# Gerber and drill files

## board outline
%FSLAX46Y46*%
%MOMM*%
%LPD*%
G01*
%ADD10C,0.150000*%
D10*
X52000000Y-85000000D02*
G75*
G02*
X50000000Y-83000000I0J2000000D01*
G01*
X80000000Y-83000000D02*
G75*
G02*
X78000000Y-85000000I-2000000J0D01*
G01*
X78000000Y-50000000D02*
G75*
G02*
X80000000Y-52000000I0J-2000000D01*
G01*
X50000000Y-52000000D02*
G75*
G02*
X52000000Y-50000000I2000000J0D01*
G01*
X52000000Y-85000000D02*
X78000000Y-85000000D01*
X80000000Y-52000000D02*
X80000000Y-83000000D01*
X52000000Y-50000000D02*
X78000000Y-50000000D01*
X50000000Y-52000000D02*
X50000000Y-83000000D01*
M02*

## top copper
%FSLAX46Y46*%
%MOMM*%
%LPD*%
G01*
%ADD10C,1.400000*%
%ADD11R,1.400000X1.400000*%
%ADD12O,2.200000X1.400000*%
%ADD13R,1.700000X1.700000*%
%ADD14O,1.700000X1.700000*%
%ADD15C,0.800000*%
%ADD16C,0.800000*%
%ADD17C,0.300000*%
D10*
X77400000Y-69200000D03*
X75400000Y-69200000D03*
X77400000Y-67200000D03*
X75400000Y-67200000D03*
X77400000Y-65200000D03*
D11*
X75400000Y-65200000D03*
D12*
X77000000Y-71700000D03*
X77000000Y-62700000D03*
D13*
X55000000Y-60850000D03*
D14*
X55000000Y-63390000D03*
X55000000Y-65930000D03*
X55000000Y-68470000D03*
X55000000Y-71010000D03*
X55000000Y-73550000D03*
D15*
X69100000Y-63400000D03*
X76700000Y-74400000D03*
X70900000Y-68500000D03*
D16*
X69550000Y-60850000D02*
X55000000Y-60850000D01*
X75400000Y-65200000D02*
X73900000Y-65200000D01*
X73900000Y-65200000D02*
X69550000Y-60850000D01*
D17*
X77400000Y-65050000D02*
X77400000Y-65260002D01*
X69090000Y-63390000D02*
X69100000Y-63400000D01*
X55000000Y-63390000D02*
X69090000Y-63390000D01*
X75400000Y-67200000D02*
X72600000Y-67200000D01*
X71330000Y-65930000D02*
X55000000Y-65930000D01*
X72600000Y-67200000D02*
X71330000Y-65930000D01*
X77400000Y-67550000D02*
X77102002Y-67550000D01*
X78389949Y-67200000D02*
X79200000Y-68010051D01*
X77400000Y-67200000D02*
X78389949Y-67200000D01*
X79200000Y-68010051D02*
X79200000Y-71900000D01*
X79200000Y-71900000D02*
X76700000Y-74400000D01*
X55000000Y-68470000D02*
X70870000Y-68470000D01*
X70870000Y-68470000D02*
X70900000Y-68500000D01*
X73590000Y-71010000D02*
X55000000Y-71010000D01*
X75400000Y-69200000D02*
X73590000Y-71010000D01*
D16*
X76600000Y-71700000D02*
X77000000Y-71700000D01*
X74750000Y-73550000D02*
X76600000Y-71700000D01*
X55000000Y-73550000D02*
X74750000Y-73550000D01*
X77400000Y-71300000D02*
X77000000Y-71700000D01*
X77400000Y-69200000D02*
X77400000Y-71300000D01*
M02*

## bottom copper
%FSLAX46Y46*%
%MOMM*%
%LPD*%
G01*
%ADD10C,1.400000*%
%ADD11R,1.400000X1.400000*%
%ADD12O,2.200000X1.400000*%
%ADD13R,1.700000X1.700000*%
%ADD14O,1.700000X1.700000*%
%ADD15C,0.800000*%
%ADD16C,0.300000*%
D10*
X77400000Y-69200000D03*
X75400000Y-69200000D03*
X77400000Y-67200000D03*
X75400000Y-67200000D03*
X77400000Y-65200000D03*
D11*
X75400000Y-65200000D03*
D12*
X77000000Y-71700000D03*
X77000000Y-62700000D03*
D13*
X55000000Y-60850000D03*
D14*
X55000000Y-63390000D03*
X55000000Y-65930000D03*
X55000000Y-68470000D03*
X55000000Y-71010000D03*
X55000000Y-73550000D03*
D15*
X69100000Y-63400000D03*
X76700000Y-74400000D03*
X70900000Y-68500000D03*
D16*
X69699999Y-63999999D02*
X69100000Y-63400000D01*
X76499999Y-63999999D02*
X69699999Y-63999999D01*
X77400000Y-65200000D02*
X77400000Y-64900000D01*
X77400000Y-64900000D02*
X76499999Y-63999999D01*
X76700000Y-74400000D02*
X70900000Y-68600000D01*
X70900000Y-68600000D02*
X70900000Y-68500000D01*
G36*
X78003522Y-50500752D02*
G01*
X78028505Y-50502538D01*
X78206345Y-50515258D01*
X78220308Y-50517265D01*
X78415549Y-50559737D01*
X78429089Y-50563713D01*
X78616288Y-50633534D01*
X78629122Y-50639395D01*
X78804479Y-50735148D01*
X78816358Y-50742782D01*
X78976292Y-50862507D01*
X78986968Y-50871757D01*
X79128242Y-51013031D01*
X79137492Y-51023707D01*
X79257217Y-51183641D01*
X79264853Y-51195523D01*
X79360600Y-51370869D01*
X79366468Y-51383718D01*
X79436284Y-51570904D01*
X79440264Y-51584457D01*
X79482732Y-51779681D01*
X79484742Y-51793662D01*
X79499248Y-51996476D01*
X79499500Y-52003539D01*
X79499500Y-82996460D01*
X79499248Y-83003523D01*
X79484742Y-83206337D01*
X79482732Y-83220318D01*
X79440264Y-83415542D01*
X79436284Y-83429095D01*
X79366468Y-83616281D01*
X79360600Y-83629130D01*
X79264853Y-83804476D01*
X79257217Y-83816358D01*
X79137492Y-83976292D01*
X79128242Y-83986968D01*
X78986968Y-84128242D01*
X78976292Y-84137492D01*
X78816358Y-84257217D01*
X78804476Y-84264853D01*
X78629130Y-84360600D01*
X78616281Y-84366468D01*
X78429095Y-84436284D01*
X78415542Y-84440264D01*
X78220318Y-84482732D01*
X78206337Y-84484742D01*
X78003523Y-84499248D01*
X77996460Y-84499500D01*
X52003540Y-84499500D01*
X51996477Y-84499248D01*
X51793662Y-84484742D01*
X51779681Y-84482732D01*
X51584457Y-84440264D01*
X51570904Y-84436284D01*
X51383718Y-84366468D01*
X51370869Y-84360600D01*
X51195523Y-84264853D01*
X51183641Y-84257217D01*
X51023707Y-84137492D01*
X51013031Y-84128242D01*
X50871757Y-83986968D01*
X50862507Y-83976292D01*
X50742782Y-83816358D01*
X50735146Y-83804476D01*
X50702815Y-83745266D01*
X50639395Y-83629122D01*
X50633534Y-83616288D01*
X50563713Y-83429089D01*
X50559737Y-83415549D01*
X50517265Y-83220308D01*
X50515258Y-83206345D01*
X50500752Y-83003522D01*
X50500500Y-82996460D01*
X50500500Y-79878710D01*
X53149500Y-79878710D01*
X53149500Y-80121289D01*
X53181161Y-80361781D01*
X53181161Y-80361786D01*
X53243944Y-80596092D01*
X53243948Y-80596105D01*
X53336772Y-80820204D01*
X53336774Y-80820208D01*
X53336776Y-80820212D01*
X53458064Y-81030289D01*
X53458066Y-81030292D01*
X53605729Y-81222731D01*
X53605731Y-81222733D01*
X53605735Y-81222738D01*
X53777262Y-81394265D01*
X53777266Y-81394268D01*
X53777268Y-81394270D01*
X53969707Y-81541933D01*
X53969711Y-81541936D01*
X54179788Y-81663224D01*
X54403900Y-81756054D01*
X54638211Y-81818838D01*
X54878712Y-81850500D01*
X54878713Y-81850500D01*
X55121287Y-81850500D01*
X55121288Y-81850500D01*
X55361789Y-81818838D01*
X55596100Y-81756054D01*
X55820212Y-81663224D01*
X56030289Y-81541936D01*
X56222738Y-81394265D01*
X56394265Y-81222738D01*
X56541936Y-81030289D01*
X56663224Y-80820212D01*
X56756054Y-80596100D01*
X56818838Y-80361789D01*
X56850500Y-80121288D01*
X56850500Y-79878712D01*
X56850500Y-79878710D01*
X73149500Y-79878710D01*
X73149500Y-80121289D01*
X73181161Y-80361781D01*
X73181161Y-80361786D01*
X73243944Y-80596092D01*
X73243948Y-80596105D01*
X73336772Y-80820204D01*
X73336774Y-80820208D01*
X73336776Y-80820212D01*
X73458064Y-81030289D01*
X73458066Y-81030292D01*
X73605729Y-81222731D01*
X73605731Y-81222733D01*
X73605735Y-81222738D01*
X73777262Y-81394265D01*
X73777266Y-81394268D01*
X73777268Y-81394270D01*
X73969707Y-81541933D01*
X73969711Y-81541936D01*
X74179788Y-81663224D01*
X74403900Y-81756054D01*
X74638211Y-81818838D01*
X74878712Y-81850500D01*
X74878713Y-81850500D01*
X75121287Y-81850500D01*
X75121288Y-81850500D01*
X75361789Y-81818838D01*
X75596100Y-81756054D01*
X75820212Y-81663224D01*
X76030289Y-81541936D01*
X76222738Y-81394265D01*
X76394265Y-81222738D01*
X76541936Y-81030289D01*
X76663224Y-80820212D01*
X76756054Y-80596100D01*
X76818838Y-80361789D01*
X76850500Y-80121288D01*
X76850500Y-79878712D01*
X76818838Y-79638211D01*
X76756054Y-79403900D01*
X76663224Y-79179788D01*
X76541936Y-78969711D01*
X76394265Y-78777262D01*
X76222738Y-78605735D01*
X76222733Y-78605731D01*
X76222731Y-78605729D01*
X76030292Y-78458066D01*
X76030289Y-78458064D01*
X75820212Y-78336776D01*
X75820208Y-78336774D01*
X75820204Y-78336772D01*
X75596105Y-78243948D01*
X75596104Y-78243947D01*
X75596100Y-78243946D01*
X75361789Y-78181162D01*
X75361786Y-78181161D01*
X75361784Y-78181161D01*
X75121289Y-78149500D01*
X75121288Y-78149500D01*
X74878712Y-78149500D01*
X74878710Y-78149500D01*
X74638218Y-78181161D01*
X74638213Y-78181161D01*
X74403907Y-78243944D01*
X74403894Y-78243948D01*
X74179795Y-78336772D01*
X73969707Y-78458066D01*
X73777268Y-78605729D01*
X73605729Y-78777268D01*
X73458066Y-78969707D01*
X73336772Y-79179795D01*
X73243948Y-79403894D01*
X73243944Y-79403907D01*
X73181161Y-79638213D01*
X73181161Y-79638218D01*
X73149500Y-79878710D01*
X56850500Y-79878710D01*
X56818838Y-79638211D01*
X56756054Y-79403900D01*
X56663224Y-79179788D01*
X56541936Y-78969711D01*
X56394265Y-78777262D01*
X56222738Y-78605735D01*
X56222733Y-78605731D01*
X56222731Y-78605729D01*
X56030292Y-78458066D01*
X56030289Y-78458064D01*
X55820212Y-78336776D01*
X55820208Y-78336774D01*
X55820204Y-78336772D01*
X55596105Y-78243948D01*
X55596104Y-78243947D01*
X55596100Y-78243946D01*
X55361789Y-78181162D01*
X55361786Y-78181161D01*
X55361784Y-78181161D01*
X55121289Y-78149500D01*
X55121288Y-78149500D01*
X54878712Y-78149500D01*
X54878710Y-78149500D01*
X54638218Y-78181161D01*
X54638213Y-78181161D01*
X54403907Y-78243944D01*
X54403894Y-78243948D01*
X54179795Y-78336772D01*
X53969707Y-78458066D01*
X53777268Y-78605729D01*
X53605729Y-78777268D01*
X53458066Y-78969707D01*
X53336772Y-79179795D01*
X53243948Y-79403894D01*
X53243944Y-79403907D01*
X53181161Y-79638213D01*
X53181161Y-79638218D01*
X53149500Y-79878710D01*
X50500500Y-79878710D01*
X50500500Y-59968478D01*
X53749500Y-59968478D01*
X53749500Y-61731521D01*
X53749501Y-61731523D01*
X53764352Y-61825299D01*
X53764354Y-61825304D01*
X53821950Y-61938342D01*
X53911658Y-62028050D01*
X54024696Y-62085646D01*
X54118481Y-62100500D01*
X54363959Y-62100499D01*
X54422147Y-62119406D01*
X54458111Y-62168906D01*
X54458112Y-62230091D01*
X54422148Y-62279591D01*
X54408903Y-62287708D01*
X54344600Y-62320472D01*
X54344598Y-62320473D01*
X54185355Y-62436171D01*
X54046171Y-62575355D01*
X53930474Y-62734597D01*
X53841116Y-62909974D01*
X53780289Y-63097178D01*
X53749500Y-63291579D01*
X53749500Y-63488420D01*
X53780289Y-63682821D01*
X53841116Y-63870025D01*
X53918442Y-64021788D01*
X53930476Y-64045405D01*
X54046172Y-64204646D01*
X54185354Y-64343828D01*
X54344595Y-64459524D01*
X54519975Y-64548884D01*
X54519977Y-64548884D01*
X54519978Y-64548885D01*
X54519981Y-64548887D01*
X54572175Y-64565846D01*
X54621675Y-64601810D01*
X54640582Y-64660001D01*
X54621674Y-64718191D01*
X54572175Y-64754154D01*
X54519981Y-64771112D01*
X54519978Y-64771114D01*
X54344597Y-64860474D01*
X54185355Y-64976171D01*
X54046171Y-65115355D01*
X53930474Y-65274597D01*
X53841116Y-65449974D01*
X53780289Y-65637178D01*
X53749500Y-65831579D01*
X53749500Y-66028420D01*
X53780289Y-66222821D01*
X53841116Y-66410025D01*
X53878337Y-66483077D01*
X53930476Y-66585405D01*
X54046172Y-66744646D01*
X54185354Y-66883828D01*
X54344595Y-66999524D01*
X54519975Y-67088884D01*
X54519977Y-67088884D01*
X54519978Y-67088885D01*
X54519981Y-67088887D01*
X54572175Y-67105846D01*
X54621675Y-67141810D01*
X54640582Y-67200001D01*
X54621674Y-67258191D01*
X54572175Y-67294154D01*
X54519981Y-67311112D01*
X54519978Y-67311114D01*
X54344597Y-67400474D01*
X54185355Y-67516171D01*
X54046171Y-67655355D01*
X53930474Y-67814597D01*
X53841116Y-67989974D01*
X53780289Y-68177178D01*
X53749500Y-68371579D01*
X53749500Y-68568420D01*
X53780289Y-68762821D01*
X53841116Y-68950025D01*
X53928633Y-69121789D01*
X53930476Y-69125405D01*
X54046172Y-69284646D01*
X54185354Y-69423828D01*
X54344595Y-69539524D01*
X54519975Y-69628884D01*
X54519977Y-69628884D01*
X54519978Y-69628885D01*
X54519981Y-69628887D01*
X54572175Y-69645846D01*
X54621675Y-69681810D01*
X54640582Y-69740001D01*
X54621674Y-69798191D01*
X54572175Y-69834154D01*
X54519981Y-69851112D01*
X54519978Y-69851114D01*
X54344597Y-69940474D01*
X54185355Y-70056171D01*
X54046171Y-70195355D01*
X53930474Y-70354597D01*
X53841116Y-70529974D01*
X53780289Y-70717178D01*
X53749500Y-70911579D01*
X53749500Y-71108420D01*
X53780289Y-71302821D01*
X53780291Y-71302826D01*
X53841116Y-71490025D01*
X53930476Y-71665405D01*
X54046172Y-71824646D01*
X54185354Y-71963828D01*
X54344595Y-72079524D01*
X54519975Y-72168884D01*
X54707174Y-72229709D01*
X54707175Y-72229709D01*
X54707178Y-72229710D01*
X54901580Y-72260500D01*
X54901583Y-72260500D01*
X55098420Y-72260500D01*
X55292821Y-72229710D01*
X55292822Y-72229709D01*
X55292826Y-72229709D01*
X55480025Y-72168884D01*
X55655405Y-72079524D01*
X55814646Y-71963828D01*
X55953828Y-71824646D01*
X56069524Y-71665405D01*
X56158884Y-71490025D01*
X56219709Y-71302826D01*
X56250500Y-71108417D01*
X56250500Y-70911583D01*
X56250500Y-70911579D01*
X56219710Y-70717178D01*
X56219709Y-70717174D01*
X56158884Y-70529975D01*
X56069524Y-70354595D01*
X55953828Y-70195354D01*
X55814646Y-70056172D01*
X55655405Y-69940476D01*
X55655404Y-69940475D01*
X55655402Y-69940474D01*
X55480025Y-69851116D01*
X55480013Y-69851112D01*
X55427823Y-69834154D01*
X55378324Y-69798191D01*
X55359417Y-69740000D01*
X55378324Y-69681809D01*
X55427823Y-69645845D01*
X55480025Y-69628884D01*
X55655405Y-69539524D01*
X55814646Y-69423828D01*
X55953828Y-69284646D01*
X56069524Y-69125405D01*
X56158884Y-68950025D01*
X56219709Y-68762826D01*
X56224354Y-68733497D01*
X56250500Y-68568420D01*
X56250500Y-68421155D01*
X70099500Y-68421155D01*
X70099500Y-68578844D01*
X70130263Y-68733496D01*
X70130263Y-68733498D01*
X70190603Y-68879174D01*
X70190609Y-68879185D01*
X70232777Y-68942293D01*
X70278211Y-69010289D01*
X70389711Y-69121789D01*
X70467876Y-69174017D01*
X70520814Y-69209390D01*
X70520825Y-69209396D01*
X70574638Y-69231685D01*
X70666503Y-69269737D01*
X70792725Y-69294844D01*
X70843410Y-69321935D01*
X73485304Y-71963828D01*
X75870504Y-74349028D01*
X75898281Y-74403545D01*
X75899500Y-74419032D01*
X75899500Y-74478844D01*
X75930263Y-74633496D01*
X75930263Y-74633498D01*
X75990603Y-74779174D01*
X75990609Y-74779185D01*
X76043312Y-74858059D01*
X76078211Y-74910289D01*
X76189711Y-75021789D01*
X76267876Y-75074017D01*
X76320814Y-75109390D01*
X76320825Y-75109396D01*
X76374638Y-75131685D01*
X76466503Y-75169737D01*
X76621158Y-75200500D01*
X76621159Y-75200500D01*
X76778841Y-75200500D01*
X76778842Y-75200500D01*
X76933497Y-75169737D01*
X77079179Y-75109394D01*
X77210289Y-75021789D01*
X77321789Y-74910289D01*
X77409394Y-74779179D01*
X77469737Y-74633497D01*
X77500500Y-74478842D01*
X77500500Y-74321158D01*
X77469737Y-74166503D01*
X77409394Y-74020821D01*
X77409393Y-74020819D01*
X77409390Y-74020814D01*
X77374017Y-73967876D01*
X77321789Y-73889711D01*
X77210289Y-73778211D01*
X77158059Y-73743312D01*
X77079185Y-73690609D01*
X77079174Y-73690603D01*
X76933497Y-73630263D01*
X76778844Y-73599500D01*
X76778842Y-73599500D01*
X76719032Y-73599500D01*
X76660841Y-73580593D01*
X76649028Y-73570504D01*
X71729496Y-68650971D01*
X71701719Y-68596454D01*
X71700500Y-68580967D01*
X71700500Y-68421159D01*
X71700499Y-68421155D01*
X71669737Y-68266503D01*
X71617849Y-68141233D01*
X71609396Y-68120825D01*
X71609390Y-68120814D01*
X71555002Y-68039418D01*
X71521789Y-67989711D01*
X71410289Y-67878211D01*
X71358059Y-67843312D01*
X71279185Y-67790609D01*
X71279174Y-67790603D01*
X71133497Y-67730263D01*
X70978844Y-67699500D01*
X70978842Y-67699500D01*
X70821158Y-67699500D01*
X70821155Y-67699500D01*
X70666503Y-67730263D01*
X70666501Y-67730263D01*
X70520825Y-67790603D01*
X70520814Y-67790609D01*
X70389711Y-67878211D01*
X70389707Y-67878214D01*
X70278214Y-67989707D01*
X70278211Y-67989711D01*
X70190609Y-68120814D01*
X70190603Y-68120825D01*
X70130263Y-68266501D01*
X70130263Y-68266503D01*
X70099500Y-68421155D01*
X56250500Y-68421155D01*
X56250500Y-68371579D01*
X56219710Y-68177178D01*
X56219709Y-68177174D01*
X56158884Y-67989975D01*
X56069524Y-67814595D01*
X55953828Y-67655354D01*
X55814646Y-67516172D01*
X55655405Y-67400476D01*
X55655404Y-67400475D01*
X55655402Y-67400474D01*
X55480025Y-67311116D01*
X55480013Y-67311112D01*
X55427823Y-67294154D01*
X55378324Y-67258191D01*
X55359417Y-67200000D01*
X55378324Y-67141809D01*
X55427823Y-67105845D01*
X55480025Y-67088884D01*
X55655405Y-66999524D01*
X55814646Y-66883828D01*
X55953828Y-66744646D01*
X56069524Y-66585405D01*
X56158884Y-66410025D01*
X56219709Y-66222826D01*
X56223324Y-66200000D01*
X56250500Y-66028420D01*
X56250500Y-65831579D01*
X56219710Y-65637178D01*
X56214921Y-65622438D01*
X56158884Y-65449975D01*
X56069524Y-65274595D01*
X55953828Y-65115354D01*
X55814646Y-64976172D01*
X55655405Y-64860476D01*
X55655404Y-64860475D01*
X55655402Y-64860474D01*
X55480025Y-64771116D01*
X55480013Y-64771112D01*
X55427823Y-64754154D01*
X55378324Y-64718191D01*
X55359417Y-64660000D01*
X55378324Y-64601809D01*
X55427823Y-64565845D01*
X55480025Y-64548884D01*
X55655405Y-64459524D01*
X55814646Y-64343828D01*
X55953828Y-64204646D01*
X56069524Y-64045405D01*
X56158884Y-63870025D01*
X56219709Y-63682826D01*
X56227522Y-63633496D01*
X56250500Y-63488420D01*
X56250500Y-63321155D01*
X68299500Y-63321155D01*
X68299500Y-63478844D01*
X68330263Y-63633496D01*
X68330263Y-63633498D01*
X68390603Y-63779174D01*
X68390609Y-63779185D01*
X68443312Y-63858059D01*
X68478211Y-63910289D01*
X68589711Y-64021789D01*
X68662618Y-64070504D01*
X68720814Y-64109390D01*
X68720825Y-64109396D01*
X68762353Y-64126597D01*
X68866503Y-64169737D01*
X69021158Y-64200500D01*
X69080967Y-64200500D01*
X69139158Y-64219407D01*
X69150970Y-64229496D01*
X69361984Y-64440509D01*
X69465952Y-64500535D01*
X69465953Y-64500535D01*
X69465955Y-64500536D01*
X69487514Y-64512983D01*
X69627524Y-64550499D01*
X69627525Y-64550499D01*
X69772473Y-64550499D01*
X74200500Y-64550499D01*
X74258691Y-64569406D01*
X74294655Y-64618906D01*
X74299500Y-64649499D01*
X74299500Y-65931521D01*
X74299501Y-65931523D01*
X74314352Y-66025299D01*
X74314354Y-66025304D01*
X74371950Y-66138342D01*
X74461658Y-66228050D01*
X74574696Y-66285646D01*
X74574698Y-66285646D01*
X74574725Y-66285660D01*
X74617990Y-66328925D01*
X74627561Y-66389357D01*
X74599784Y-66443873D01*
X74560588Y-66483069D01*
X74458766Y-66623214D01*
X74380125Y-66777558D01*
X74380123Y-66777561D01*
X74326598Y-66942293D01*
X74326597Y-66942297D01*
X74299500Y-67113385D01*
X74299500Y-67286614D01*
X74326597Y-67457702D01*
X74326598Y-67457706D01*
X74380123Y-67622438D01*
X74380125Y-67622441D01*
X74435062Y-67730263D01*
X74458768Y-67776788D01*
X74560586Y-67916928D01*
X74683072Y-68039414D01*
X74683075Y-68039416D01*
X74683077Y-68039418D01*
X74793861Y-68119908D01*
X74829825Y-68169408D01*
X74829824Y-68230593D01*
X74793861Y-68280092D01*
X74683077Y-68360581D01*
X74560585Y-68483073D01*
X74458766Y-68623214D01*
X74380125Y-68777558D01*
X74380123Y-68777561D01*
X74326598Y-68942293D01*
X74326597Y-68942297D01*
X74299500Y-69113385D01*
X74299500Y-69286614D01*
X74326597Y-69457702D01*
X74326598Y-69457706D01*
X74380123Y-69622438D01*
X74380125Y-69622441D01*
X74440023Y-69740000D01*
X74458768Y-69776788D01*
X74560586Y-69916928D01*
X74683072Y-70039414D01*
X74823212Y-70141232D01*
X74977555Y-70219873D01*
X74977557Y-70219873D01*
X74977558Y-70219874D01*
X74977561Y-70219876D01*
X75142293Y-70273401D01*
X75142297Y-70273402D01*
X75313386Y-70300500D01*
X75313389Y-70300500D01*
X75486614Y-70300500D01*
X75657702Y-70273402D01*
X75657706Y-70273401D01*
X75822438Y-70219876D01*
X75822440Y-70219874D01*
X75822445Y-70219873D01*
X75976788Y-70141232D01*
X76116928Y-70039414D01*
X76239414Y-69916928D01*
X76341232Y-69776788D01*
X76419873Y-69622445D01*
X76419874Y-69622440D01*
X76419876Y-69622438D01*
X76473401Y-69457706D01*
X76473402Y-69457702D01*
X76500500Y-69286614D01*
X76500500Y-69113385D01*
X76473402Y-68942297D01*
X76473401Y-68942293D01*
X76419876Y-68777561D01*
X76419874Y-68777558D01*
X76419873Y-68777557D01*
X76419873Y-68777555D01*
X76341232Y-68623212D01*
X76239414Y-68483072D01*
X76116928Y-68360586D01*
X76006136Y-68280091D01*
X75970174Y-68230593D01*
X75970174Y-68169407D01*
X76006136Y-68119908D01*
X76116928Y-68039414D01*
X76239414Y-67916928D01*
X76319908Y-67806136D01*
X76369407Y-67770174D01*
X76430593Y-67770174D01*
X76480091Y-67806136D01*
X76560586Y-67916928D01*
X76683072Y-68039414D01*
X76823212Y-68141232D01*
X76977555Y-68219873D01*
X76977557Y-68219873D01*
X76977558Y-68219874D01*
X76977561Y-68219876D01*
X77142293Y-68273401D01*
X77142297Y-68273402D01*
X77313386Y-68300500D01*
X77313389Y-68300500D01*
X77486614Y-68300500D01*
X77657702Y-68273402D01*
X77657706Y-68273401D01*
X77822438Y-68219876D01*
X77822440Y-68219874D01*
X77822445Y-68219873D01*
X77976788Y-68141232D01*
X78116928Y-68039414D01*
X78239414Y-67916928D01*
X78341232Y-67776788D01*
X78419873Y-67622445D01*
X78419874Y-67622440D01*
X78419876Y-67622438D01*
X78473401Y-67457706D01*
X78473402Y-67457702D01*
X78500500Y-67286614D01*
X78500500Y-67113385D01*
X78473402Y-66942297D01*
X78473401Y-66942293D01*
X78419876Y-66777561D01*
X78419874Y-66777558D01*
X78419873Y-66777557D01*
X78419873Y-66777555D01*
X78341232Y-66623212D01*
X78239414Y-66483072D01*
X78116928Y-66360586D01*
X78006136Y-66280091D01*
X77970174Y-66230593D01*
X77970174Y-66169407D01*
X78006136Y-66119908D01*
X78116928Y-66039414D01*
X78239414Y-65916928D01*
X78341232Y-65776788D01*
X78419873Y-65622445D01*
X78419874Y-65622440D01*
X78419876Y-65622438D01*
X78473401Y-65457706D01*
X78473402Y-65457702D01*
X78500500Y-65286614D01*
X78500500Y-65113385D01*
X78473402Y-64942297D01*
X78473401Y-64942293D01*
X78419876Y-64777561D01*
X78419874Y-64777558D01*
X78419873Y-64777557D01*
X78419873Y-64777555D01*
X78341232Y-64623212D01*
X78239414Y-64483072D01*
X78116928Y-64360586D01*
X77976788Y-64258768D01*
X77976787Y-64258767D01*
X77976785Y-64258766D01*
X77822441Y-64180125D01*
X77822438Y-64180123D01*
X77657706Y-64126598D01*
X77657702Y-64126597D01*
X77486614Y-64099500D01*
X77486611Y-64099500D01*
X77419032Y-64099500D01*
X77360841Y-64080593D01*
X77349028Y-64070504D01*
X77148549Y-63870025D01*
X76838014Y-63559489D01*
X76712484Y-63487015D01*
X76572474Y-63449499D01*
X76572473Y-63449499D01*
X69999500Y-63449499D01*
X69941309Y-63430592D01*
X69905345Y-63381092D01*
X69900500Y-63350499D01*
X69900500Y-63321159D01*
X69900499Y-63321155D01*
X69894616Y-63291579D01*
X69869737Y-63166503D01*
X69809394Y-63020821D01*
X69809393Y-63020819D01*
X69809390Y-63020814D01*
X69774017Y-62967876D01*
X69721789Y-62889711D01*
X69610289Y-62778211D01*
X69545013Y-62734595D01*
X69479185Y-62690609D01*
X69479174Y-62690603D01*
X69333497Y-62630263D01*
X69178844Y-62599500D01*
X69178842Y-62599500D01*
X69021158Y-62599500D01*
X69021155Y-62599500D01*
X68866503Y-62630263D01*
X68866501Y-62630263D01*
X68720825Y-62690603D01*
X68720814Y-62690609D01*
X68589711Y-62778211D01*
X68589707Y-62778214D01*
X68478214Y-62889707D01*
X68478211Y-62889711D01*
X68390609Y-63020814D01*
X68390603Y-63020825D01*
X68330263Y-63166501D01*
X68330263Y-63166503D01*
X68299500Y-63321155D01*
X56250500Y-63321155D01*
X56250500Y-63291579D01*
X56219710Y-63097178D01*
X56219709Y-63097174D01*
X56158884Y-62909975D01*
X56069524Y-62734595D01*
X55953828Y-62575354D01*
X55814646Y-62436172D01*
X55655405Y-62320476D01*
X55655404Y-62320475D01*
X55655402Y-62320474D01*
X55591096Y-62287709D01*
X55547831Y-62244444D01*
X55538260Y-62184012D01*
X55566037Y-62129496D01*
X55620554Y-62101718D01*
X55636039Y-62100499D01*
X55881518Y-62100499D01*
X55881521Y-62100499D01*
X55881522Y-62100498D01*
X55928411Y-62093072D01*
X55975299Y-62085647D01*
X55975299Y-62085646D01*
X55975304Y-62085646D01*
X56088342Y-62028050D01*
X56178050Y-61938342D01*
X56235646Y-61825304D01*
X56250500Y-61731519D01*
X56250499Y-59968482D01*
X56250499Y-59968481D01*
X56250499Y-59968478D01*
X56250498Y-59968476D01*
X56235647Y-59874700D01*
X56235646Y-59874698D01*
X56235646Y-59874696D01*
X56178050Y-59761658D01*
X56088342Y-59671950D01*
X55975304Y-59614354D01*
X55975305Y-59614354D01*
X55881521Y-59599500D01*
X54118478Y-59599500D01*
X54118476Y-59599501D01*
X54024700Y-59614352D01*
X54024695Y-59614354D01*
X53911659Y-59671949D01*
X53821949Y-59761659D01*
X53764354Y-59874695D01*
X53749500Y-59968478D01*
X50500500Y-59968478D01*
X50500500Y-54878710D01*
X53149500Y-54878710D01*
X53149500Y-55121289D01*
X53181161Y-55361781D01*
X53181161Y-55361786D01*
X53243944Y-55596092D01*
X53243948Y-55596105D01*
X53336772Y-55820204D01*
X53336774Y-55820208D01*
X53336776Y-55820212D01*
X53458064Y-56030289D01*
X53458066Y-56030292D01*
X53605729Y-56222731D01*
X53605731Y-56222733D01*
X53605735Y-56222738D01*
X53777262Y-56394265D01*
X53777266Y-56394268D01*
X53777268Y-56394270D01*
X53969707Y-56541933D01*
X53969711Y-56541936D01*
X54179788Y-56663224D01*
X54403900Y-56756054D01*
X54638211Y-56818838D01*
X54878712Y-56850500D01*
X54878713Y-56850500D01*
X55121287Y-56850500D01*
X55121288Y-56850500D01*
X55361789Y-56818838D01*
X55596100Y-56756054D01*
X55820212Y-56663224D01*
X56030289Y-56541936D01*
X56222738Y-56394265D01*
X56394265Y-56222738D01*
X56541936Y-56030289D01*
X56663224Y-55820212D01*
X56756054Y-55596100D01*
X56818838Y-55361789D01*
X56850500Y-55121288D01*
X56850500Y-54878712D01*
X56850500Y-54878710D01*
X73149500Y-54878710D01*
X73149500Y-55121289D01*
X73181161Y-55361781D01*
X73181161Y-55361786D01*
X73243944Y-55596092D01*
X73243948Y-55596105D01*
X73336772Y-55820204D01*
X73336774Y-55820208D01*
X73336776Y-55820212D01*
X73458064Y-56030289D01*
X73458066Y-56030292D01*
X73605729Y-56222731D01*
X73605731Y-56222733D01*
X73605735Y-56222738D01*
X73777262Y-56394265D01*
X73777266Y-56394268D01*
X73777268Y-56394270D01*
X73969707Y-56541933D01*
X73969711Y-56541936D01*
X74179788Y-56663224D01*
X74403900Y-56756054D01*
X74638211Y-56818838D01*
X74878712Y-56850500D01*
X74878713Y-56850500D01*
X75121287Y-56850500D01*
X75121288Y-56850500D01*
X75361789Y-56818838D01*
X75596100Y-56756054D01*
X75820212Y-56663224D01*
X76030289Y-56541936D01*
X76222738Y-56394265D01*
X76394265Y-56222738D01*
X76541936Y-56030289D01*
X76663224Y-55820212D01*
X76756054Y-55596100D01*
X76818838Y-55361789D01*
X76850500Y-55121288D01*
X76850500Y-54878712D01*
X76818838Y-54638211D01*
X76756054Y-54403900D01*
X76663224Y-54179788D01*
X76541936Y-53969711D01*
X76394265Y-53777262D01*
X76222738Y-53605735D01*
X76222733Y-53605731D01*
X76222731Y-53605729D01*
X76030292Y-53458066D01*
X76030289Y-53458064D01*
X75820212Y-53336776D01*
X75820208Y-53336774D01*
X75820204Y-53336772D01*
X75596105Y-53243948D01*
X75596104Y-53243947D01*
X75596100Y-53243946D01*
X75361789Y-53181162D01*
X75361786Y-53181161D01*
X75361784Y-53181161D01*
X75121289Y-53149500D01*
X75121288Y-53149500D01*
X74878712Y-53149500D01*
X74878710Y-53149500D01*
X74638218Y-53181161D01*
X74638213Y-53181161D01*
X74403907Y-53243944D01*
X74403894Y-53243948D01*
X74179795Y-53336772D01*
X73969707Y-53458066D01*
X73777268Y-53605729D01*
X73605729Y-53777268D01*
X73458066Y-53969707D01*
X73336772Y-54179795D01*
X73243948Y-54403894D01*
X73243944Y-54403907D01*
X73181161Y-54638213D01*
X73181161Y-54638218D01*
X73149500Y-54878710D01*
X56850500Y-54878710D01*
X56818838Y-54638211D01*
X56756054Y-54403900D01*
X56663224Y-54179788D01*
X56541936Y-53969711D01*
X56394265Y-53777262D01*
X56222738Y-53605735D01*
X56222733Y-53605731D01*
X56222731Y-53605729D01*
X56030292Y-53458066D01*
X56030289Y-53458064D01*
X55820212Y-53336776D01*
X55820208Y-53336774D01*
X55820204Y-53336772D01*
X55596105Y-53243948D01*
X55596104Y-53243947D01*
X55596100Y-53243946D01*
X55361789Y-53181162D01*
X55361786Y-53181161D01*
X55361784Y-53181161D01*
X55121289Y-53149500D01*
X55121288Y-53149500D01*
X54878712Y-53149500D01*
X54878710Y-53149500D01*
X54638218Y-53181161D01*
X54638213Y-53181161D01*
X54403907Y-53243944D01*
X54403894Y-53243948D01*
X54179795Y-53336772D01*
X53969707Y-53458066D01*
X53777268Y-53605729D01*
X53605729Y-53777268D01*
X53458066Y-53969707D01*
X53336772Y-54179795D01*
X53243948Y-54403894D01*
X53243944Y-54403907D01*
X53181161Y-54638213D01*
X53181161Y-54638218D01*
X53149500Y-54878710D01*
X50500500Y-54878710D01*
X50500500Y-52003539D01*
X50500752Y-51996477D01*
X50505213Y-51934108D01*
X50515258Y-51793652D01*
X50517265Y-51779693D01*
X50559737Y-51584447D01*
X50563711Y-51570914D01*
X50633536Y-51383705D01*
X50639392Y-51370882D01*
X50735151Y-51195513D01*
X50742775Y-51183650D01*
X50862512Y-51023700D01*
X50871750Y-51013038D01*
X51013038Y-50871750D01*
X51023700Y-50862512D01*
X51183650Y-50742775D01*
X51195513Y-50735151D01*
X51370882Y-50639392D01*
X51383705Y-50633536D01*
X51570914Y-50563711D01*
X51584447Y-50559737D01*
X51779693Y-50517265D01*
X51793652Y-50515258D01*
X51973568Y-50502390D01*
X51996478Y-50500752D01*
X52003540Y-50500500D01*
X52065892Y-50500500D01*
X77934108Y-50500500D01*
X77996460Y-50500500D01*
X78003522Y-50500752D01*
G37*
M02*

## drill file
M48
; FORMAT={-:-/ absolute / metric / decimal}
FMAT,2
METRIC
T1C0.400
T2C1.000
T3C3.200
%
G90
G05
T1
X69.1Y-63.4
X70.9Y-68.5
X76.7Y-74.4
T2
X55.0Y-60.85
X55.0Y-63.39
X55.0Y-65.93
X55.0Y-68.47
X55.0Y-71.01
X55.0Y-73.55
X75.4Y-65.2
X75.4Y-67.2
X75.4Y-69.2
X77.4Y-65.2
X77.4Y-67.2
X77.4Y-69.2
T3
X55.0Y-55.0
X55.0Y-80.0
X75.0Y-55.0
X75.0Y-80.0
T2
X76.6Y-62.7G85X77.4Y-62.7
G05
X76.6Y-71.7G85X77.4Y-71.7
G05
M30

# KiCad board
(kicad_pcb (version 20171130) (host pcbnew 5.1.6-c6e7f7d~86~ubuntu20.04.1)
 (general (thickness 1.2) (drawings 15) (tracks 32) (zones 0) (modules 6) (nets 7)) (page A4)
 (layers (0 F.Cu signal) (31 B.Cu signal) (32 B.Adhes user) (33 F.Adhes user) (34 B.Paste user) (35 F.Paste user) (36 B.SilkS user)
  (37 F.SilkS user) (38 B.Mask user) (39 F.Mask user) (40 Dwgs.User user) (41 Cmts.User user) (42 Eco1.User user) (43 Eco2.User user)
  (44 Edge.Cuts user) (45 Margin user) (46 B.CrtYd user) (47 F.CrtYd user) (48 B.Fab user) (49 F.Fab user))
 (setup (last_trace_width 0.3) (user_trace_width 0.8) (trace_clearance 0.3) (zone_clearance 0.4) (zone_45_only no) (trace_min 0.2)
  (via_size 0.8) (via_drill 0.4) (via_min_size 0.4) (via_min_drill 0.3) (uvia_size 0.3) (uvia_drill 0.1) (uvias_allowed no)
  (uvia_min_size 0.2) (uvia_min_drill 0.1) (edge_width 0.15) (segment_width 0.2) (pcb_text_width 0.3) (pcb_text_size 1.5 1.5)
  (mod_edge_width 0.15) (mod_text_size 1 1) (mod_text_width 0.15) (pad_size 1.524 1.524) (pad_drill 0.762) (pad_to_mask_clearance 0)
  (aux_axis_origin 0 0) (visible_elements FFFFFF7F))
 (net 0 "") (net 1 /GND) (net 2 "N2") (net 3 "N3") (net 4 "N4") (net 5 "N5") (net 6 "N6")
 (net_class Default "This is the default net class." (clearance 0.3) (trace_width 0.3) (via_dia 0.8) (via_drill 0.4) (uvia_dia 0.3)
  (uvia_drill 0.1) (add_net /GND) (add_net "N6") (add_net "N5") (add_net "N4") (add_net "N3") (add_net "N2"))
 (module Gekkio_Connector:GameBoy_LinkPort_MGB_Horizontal (layer F.Cu) (at 75.4 65.2)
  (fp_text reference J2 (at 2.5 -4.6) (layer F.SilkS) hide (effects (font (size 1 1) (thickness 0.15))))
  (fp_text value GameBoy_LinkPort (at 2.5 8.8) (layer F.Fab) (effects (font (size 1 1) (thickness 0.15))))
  (pad 6 thru_hole circle (at 2 4) (size 1.4 1.4) (drill 1) (layers *.Cu *.Mask) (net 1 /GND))
  (pad 5 thru_hole circle (at 0 4) (size 1.4 1.4) (drill 1) (layers *.Cu *.Mask) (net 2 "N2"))
  (pad 4 thru_hole circle (at 2 2) (size 1.4 1.4) (drill 1) (layers *.Cu *.Mask) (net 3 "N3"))
  (pad 3 thru_hole circle (at 0 2) (size 1.4 1.4) (drill 1) (layers *.Cu *.Mask) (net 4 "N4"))
  (pad 2 thru_hole circle (at 2 0) (size 1.4 1.4) (drill 1) (layers *.Cu *.Mask) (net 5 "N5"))
  (pad 1 thru_hole rect (at 0 0) (size 1.4 1.4) (drill 1) (layers *.Cu *.Mask) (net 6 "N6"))
  (pad SH thru_hole oval (at 1.6 6.5 90) (size 1.4 2.2) (drill oval 1 1.8) (layers *.Cu *.Mask) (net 1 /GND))
  (pad SH thru_hole oval (at 1.6 -2.5 90) (size 1.4 2.2) (drill oval 1 1.8) (layers *.Cu *.Mask) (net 1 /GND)))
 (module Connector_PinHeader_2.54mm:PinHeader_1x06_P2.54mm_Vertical (layer F.Cu) (at 55 60.85)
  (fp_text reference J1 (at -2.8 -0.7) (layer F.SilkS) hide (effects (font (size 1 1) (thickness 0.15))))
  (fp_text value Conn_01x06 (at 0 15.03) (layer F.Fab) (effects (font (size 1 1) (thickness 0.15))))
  (pad 1 thru_hole rect (at 0 0) (size 1.7 1.7) (drill 1) (layers *.Cu *.Mask) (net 6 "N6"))
  (pad 2 thru_hole oval (at 0 2.54) (size 1.7 1.7) (drill 1) (layers *.Cu *.Mask) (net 5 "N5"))
  (pad 3 thru_hole oval (at 0 5.08) (size 1.7 1.7) (drill 1) (layers *.Cu *.Mask) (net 4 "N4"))
  (pad 4 thru_hole oval (at 0 7.62) (size 1.7 1.7) (drill 1) (layers *.Cu *.Mask) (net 3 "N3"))
  (pad 5 thru_hole oval (at 0 10.16) (size 1.7 1.7) (drill 1) (layers *.Cu *.Mask) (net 2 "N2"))
  (pad 6 thru_hole oval (at 0 12.7) (size 1.7 1.7) (drill 1) (layers *.Cu *.Mask) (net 1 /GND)))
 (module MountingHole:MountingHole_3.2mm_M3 (layer F.Cu) (at 75 80)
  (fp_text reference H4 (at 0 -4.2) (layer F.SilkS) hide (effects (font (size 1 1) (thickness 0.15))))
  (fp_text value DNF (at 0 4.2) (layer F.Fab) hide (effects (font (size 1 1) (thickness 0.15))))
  (pad 1 np_thru_hole circle (at 0 0) (size 3.2 3.2) (drill 3.2) (layers *.Cu *.Mask)))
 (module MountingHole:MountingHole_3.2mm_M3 (layer F.Cu) (at 75 55)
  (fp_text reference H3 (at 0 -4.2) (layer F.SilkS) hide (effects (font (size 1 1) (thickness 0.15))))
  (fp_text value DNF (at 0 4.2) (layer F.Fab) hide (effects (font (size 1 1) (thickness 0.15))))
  (pad 1 np_thru_hole circle (at 0 0) (size 3.2 3.2) (drill 3.2) (layers *.Cu *.Mask)))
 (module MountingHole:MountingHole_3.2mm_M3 (layer F.Cu) (at 55 80)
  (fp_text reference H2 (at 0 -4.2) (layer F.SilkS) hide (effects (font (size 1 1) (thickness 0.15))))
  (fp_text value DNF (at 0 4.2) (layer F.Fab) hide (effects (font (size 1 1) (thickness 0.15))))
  (pad 1 np_thru_hole circle (at 0 0) (size 3.2 3.2) (drill 3.2) (layers *.Cu *.Mask)))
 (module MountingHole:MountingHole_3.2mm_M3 (layer F.Cu) (at 55 55)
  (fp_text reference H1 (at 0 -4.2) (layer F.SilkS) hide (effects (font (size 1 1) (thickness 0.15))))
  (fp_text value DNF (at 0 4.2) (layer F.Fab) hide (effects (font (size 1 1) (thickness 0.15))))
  (pad 1 np_thru_hole circle (at 0 0) (size 3.2 3.2) (drill 3.2) (layers *.Cu *.Mask)))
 (gr_arc (start 52 83) (end 50 83) (angle -90) (layer Edge.Cuts) (width 0.15))
 (gr_arc (start 78 83) (end 78 85) (angle -90) (layer Edge.Cuts) (width 0.15))
 (gr_arc (start 78 52) (end 80 52) (angle -90) (layer Edge.Cuts) (width 0.15))
 (gr_arc (start 52 52) (end 52 50) (angle -90) (layer Edge.Cuts) (width 0.15))
 (gr_line (start 52 85) (end 78 85) (layer Edge.Cuts) (width 0.15))
 (gr_line (start 80 52) (end 80 83) (layer Edge.Cuts) (width 0.15))
 (gr_line (start 52 50) (end 78 50) (layer Edge.Cuts) (width 0.15))
 (gr_line (start 50 52) (end 50 83) (layer Edge.Cuts) (width 0.15))
 (segment (start 69.55 60.85) (end 55 60.85) (width 0.8) (layer F.Cu) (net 6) (status 20))
 (segment (start 75.4 65.2) (end 73.9 65.2) (width 0.8) (layer F.Cu) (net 6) (status 10))
 (segment (start 73.9 65.2) (end 69.55 60.85) (width 0.8) (layer F.Cu) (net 6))
 (segment (start 77.4 65.05) (end 77.4 65.260002) (width 0.3) (layer F.Cu) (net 5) (status 30))
 (segment (start 69.09 63.39) (end 69.1 63.4) (width 0.3) (layer F.Cu) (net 5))
 (segment (start 55 63.39) (end 69.09 63.39) (width 0.3) (layer F.Cu) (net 5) (status 10))
 (via (at 69.1 63.4) (size 0.8) (drill 0.4) (layers F.Cu B.Cu) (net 5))
 (segment (start 69.699999 63.999999) (end 69.1 63.4) (width 0.3) (layer B.Cu) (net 5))
 (segment (start 76.499999 63.999999) (end 69.699999 63.999999) (width 0.3) (layer B.Cu) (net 5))
 (segment (start 77.4 65.2) (end 77.4 64.9) (width 0.3) (layer B.Cu) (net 5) (status 30))
 (segment (start 77.4 64.9) (end 76.499999 63.999999) (width 0.3) (layer B.Cu) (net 5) (status 10))
 (segment (start 75.4 67.2) (end 72.6 67.2) (width 0.3) (layer F.Cu) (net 4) (status 10))
 (segment (start 71.33 65.93) (end 55 65.93) (width 0.3) (layer F.Cu) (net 4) (status 20))
 (segment (start 72.6 67.2) (end 71.33 65.93) (width 0.3) (layer F.Cu) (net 4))
 (segment (start 77.4 67.55) (end 77.102002 67.55) (width 0.3) (layer F.Cu) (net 3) (status 30))
 (segment (start 78.389949 67.2) (end 79.2 68.010051) (width 0.3) (layer F.Cu) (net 3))
 (segment (start 77.4 67.2) (end 78.389949 67.2) (width 0.3) (layer F.Cu) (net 3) (status 10))
 (via (at 76.7 74.4) (size 0.8) (drill 0.4) (layers F.Cu B.Cu) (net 3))
 (segment (start 79.2 68.010051) (end 79.2 71.9) (width 0.3) (layer F.Cu) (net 3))
 (segment (start 79.2 71.9) (end 76.7 74.4) (width 0.3) (layer F.Cu) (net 3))
 (segment (start 76.7 74.4) (end 70.9 68.6) (width 0.3) (layer B.Cu) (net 3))
 (segment (start 70.9 68.6) (end 70.9 68.5) (width 0.3) (layer B.Cu) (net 3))
 (via (at 70.9 68.5) (size 0.8) (drill 0.4) (layers F.Cu B.Cu) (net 3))
 (segment (start 55 68.47) (end 70.87 68.47) (width 0.3) (layer F.Cu) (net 3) (status 10))
 (segment (start 70.87 68.47) (end 70.9 68.5) (width 0.3) (layer F.Cu) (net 3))
 (segment (start 73.59 71.01) (end 55 71.01) (width 0.3) (layer F.Cu) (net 2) (status 20))
 (segment (start 75.4 69.2) (end 73.59 71.01) (width 0.3) (layer F.Cu) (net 2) (status 10))
 (segment (start 76.6 71.7) (end 77 71.7) (width 0.8) (layer F.Cu) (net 1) (status 30))
 (segment (start 74.75 73.55) (end 76.6 71.7) (width 0.8) (layer F.Cu) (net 1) (status 20))
 (segment (start 55 73.55) (end 74.75 73.55) (width 0.8) (layer F.Cu) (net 1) (status 10))
 (segment (start 77.4 71.3) (end 77 71.7) (width 0.8) (layer F.Cu) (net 1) (status 30))
 (segment (start 77.4 69.2) (end 77.4 71.3) (width 0.8) (layer F.Cu) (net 1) (status 30))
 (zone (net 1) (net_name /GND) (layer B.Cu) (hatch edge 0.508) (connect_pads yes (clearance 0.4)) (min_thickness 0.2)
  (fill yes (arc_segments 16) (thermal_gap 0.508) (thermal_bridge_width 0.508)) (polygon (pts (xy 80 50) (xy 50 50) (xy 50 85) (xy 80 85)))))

